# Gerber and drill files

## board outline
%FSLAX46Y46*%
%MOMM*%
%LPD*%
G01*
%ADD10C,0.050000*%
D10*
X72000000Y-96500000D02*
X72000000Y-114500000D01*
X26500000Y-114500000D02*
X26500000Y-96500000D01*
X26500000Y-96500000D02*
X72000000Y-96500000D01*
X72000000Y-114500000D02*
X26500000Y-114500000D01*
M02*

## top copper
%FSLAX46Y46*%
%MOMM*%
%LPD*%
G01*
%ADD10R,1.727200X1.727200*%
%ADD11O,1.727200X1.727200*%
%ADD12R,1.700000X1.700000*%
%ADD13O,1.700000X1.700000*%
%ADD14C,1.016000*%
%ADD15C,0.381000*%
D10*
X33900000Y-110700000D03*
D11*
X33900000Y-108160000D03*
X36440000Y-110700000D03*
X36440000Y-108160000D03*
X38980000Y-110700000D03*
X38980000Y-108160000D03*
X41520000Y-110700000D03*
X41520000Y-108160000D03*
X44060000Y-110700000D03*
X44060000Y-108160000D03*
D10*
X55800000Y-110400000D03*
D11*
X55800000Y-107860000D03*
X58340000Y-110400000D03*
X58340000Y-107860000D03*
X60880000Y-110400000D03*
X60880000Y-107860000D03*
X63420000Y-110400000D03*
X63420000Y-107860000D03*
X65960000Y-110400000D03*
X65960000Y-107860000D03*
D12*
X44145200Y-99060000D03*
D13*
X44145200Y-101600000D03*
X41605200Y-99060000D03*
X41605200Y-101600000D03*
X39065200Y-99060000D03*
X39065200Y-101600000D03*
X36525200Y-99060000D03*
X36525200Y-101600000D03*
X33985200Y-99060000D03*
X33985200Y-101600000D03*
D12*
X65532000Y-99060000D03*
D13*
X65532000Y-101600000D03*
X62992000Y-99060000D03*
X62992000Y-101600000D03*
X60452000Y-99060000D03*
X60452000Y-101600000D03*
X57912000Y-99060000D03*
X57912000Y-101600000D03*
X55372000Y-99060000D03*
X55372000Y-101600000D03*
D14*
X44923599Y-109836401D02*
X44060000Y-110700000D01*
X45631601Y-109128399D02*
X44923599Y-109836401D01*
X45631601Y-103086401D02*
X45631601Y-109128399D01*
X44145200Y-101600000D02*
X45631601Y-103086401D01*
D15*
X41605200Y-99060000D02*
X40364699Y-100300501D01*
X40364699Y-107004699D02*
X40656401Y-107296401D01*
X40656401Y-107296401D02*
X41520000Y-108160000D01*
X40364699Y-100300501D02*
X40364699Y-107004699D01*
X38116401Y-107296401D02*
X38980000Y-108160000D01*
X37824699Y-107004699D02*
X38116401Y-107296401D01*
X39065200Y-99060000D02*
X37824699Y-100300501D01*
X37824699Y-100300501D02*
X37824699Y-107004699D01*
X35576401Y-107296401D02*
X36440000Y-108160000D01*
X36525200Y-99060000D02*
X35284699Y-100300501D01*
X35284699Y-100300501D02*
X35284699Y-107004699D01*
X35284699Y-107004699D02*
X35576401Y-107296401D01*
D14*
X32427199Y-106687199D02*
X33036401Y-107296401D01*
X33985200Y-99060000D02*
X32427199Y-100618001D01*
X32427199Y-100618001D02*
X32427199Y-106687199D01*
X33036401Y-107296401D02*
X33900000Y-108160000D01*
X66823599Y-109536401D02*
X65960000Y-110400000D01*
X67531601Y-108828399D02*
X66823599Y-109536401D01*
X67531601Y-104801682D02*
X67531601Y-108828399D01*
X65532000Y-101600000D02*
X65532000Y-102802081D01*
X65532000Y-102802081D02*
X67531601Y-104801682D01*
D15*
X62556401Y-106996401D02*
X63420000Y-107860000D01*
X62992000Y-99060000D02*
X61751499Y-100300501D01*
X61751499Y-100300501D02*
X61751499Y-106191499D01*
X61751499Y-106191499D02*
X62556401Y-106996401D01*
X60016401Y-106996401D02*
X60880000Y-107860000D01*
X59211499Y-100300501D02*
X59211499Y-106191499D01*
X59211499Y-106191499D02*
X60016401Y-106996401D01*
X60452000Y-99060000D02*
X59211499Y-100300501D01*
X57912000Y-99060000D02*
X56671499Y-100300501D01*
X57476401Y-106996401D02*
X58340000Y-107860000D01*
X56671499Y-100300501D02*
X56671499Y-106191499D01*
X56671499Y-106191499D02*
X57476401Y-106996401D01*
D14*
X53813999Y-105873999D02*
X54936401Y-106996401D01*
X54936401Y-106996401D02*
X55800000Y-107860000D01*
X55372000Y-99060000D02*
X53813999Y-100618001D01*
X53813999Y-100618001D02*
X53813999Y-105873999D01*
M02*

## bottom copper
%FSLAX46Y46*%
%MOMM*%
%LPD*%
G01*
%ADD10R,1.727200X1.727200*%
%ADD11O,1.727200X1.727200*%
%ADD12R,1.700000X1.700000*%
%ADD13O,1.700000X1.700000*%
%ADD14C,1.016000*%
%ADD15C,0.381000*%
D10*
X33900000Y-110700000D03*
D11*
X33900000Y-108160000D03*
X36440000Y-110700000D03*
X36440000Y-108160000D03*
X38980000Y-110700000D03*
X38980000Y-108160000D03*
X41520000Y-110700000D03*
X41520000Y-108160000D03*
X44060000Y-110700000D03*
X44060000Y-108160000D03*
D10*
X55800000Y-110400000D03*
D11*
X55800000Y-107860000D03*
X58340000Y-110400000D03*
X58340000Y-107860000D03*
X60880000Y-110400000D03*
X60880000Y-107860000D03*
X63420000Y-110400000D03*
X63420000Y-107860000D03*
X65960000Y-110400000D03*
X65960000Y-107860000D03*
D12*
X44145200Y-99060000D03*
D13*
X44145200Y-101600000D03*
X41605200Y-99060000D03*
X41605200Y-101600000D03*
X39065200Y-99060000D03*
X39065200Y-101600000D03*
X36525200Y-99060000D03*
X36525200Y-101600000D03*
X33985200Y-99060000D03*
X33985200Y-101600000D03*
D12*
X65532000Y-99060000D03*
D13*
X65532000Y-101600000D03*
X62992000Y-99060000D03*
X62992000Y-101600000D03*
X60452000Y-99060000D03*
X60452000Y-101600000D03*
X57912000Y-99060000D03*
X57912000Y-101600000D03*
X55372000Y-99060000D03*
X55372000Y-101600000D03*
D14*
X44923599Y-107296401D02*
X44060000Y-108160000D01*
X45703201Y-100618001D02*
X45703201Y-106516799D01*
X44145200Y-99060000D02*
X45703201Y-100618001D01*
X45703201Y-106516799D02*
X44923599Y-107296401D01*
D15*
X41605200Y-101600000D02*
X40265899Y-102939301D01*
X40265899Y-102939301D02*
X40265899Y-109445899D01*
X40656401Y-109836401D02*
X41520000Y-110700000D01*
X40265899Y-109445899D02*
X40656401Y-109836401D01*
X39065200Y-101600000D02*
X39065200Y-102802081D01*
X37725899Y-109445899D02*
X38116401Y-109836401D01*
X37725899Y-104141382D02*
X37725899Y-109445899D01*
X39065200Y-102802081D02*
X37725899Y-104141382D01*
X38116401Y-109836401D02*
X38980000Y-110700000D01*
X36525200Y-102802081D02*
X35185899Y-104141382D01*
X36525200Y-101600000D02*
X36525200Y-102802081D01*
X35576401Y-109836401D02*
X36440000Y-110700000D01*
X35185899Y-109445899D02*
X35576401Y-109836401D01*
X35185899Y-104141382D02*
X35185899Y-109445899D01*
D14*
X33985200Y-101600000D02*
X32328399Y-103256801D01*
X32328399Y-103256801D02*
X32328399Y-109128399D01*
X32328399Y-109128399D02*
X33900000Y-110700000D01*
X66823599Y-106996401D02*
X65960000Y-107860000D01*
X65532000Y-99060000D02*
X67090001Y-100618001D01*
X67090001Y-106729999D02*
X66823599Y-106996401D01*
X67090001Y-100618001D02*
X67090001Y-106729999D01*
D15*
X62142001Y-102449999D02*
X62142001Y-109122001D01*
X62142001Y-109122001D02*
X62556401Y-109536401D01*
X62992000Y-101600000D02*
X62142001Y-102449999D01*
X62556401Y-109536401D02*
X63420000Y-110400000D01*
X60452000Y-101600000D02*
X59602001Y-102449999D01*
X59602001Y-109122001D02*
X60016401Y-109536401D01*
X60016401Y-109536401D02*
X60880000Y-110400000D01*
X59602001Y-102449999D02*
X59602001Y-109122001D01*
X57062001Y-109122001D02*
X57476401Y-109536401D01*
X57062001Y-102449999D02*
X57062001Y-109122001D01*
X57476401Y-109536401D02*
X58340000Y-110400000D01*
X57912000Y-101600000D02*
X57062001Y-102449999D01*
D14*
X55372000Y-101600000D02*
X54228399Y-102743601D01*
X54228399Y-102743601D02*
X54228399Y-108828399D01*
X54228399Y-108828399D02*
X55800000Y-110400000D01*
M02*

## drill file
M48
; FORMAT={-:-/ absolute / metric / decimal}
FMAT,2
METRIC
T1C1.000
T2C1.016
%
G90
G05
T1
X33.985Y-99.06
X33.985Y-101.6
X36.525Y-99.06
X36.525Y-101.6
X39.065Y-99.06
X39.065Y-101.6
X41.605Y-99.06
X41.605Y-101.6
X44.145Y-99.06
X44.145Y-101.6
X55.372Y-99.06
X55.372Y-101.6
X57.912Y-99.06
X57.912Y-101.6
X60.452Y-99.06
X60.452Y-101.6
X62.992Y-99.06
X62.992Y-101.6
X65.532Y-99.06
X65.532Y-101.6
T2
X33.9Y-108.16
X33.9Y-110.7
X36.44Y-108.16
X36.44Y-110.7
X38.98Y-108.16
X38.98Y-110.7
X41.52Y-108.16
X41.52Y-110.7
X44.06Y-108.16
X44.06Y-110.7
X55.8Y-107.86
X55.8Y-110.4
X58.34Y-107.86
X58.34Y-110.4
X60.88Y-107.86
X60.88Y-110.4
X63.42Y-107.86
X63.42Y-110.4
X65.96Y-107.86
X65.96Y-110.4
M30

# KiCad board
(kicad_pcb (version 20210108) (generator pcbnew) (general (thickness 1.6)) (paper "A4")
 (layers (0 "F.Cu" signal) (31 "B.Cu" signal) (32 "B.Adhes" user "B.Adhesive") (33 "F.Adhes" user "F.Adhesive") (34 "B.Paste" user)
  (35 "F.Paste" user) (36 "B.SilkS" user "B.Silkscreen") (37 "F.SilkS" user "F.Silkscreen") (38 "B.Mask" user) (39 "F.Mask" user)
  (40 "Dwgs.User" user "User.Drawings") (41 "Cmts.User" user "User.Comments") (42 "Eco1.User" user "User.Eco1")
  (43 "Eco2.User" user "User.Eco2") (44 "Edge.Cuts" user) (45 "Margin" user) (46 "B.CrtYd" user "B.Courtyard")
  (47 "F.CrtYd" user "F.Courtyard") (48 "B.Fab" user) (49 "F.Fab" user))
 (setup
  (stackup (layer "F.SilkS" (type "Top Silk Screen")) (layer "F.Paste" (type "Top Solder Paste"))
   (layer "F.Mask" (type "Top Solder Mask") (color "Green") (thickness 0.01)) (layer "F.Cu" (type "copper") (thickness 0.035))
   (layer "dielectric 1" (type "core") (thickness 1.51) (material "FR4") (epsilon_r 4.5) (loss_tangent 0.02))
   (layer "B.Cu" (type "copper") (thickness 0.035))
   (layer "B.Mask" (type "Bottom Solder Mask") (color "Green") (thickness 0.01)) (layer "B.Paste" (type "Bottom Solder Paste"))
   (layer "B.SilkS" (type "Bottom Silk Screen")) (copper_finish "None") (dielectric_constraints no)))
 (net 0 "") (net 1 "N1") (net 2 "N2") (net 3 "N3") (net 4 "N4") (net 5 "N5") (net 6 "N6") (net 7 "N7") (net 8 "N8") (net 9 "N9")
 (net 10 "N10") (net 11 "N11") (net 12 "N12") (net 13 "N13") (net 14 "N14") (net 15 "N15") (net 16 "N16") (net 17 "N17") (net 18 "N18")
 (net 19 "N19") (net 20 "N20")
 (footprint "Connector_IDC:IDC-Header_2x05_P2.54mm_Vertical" (layer "F.Cu") (at 33.9 110.7 90)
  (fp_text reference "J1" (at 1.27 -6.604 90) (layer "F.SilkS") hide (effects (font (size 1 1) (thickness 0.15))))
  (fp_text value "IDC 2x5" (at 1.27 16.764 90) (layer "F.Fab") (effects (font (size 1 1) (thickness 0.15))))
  (pad "1" thru_hole rect (at 0 0 90) (locked) (size 1.7272 1.7272) (drill 1.016) (layers *.Cu *.Mask) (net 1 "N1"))
  (pad "2" thru_hole oval (at 2.54 0 90) (locked) (size 1.7272 1.7272) (drill 1.016) (layers *.Cu *.Mask) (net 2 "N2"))
  (pad "3" thru_hole oval (at 0 2.54 90) (locked) (size 1.7272 1.7272) (drill 1.016) (layers *.Cu *.Mask) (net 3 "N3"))
  (pad "4" thru_hole oval (at 2.54 2.54 90) (locked) (size 1.7272 1.7272) (drill 1.016) (layers *.Cu *.Mask) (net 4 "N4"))
  (pad "5" thru_hole oval (at 0 5.08 90) (locked) (size 1.7272 1.7272) (drill 1.016) (layers *.Cu *.Mask) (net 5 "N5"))
  (pad "6" thru_hole oval (at 2.54 5.08 90) (locked) (size 1.7272 1.7272) (drill 1.016) (layers *.Cu *.Mask) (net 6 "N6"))
  (pad "7" thru_hole oval (at 0 7.62 90) (locked) (size 1.7272 1.7272) (drill 1.016) (layers *.Cu *.Mask) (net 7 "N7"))
  (pad "8" thru_hole oval (at 2.54 7.62 90) (locked) (size 1.7272 1.7272) (drill 1.016) (layers *.Cu *.Mask) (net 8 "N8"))
  (pad "9" thru_hole oval (at 0 10.16 90) (locked) (size 1.7272 1.7272) (drill 1.016) (layers *.Cu *.Mask) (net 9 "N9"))
  (pad "10" thru_hole oval (at 2.54 10.16 90) (locked) (size 1.7272 1.7272) (drill 1.016) (layers *.Cu *.Mask) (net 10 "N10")))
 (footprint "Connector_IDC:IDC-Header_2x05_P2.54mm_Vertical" (layer "F.Cu") (at 55.8 110.4 90)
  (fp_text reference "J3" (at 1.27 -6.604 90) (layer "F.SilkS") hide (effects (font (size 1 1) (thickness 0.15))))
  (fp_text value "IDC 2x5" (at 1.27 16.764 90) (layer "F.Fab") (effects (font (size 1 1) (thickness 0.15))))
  (pad "1" thru_hole rect (at 0 0 90) (locked) (size 1.7272 1.7272) (drill 1.016) (layers *.Cu *.Mask) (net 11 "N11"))
  (pad "2" thru_hole oval (at 2.54 0 90) (locked) (size 1.7272 1.7272) (drill 1.016) (layers *.Cu *.Mask) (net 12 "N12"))
  (pad "3" thru_hole oval (at 0 2.54 90) (locked) (size 1.7272 1.7272) (drill 1.016) (layers *.Cu *.Mask) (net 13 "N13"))
  (pad "4" thru_hole oval (at 2.54 2.54 90) (locked) (size 1.7272 1.7272) (drill 1.016) (layers *.Cu *.Mask) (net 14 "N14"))
  (pad "5" thru_hole oval (at 0 5.08 90) (locked) (size 1.7272 1.7272) (drill 1.016) (layers *.Cu *.Mask) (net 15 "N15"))
  (pad "6" thru_hole oval (at 2.54 5.08 90) (locked) (size 1.7272 1.7272) (drill 1.016) (layers *.Cu *.Mask) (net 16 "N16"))
  (pad "7" thru_hole oval (at 0 7.62 90) (locked) (size 1.7272 1.7272) (drill 1.016) (layers *.Cu *.Mask) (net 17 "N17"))
  (pad "8" thru_hole oval (at 2.54 7.62 90) (locked) (size 1.7272 1.7272) (drill 1.016) (layers *.Cu *.Mask) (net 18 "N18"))
  (pad "9" thru_hole oval (at 0 10.16 90) (locked) (size 1.7272 1.7272) (drill 1.016) (layers *.Cu *.Mask) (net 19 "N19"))
  (pad "10" thru_hole oval (at 2.54 10.16 90) (locked) (size 1.7272 1.7272) (drill 1.016) (layers *.Cu *.Mask) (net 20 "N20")))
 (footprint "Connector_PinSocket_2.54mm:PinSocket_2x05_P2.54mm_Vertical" (layer "B.Cu") (at 44.1452 99.06 90)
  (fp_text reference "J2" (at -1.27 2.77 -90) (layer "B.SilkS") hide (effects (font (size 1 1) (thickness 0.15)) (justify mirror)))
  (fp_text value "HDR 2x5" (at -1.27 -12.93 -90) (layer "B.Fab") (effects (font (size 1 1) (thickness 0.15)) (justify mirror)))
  (pad "1" thru_hole rect (at 0 0 90) (locked) (size 1.7 1.7) (drill 1) (layers *.Cu *.Mask) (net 10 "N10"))
  (pad "2" thru_hole oval (at -2.54 0 90) (locked) (size 1.7 1.7) (drill 1) (layers *.Cu *.Mask) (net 9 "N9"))
  (pad "3" thru_hole oval (at 0 -2.54 90) (locked) (size 1.7 1.7) (drill 1) (layers *.Cu *.Mask) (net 8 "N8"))
  (pad "4" thru_hole oval (at -2.54 -2.54 90) (locked) (size 1.7 1.7) (drill 1) (layers *.Cu *.Mask) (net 7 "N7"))
  (pad "5" thru_hole oval (at 0 -5.08 90) (locked) (size 1.7 1.7) (drill 1) (layers *.Cu *.Mask) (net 6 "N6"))
  (pad "6" thru_hole oval (at -2.54 -5.08 90) (locked) (size 1.7 1.7) (drill 1) (layers *.Cu *.Mask) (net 5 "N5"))
  (pad "7" thru_hole oval (at 0 -7.62 90) (locked) (size 1.7 1.7) (drill 1) (layers *.Cu *.Mask) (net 4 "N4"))
  (pad "8" thru_hole oval (at -2.54 -7.62 90) (locked) (size 1.7 1.7) (drill 1) (layers *.Cu *.Mask) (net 3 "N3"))
  (pad "9" thru_hole oval (at 0 -10.16 90) (locked) (size 1.7 1.7) (drill 1) (layers *.Cu *.Mask) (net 2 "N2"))
  (pad "10" thru_hole oval (at -2.54 -10.16 90) (locked) (size 1.7 1.7) (drill 1) (layers *.Cu *.Mask) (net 1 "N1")))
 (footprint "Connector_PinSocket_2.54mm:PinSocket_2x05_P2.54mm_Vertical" (layer "B.Cu") (at 65.532 99.06 90)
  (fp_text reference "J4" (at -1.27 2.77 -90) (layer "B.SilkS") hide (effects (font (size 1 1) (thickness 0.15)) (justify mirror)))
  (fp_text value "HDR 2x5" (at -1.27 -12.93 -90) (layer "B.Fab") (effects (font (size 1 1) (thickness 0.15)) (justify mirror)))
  (pad "1" thru_hole rect (at 0 0 90) (locked) (size 1.7 1.7) (drill 1) (layers *.Cu *.Mask) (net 20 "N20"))
  (pad "2" thru_hole oval (at -2.54 0 90) (locked) (size 1.7 1.7) (drill 1) (layers *.Cu *.Mask) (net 19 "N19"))
  (pad "3" thru_hole oval (at 0 -2.54 90) (locked) (size 1.7 1.7) (drill 1) (layers *.Cu *.Mask) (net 18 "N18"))
  (pad "4" thru_hole oval (at -2.54 -2.54 90) (locked) (size 1.7 1.7) (drill 1) (layers *.Cu *.Mask) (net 17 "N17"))
  (pad "5" thru_hole oval (at 0 -5.08 90) (locked) (size 1.7 1.7) (drill 1) (layers *.Cu *.Mask) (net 16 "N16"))
  (pad "6" thru_hole oval (at -2.54 -5.08 90) (locked) (size 1.7 1.7) (drill 1) (layers *.Cu *.Mask) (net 15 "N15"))
  (pad "7" thru_hole oval (at 0 -7.62 90) (locked) (size 1.7 1.7) (drill 1) (layers *.Cu *.Mask) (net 14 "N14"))
  (pad "8" thru_hole oval (at -2.54 -7.62 90) (locked) (size 1.7 1.7) (drill 1) (layers *.Cu *.Mask) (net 13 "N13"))
  (pad "9" thru_hole oval (at 0 -10.16 90) (locked) (size 1.7 1.7) (drill 1) (layers *.Cu *.Mask) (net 12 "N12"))
  (pad "10" thru_hole oval (at -2.54 -10.16 90) (locked) (size 1.7 1.7) (drill 1) (layers *.Cu *.Mask) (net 11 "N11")))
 (gr_line (start 72 96.5) (end 72 114.5) (layer "Edge.Cuts") (width 0.05))
 (gr_line (start 26.5 114.5) (end 26.5 96.5) (layer "Edge.Cuts") (width 0.05))
 (gr_line (start 26.5 96.5) (end 72 96.5) (layer "Edge.Cuts") (width 0.05))
 (gr_line (start 72 114.5) (end 26.5 114.5) (layer "Edge.Cuts") (width 0.05))
 (segment (start 44.923599 107.296401) (end 44.06 108.16) (width 1.016) (layer "B.Cu") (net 10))
 (segment (start 45.703201 100.618001) (end 45.703201 106.516799) (width 1.016) (layer "B.Cu") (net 10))
 (segment (start 44.1452 99.06) (end 45.703201 100.618001) (width 1.016) (layer "B.Cu") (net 10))
 (segment (start 45.703201 106.516799) (end 44.923599 107.296401) (width 1.016) (layer "B.Cu") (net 10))
 (segment (start 44.923599 109.836401) (end 44.06 110.7) (width 1.016) (layer "F.Cu") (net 9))
 (segment (start 45.631601 109.128399) (end 44.923599 109.836401) (width 1.016) (layer "F.Cu") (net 9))
 (segment (start 45.631601 103.086401) (end 45.631601 109.128399) (width 1.016) (layer "F.Cu") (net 9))
 (segment (start 44.1452 101.6) (end 45.631601 103.086401) (width 1.016) (layer "F.Cu") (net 9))
 (segment (start 41.6052 99.06) (end 40.364699 100.300501) (width 0.381) (layer "F.Cu") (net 8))
 (segment (start 40.364699 107.004699) (end 40.656401 107.296401) (width 0.381) (layer "F.Cu") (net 8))
 (segment (start 40.656401 107.296401) (end 41.52 108.16) (width 0.381) (layer "F.Cu") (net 8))
 (segment (start 40.364699 100.300501) (end 40.364699 107.004699) (width 0.381) (layer "F.Cu") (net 8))
 (segment (start 41.6052 101.6) (end 40.265899 102.939301) (width 0.381) (layer "B.Cu") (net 7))
 (segment (start 40.265899 102.939301) (end 40.265899 109.445899) (width 0.381) (layer "B.Cu") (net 7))
 (segment (start 40.656401 109.836401) (end 41.52 110.7) (width 0.381) (layer "B.Cu") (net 7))
 (segment (start 40.265899 109.445899) (end 40.656401 109.836401) (width 0.381) (layer "B.Cu") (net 7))
 (segment (start 38.116401 107.296401) (end 38.98 108.16) (width 0.381) (layer "F.Cu") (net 6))
 (segment (start 37.824699 107.004699) (end 38.116401 107.296401) (width 0.381) (layer "F.Cu") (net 6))
 (segment (start 39.0652 99.06) (end 37.824699 100.300501) (width 0.381) (layer "F.Cu") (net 6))
 (segment (start 37.824699 100.300501) (end 37.824699 107.004699) (width 0.381) (layer "F.Cu") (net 6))
 (segment (start 39.0652 101.6) (end 39.0652 102.802081) (width 0.381) (layer "B.Cu") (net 5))
 (segment (start 37.725899 109.445899) (end 38.116401 109.836401) (width 0.381) (layer "B.Cu") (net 5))
 (segment (start 37.725899 104.141382) (end 37.725899 109.445899) (width 0.381) (layer "B.Cu") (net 5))
 (segment (start 39.0652 102.802081) (end 37.725899 104.141382) (width 0.381) (layer "B.Cu") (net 5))
 (segment (start 38.116401 109.836401) (end 38.98 110.7) (width 0.381) (layer "B.Cu") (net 5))
 (segment (start 35.576401 107.296401) (end 36.44 108.16) (width 0.381) (layer "F.Cu") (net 4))
 (segment (start 36.5252 99.06) (end 35.284699 100.300501) (width 0.381) (layer "F.Cu") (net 4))
 (segment (start 35.284699 100.300501) (end 35.284699 107.004699) (width 0.381) (layer "F.Cu") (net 4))
 (segment (start 35.284699 107.004699) (end 35.576401 107.296401) (width 0.381) (layer "F.Cu") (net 4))
 (segment (start 36.5252 102.802081) (end 35.185899 104.141382) (width 0.381) (layer "B.Cu") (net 3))
 (segment (start 36.5252 101.6) (end 36.5252 102.802081) (width 0.381) (layer "B.Cu") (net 3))
 (segment (start 35.576401 109.836401) (end 36.44 110.7) (width 0.381) (layer "B.Cu") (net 3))
 (segment (start 35.185899 109.445899) (end 35.576401 109.836401) (width 0.381) (layer "B.Cu") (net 3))
 (segment (start 35.185899 104.141382) (end 35.185899 109.445899) (width 0.381) (layer "B.Cu") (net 3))
 (segment (start 32.427199 106.687199) (end 33.036401 107.296401) (width 1.016) (layer "F.Cu") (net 2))
 (segment (start 33.9852 99.06) (end 32.427199 100.618001) (width 1.016) (layer "F.Cu") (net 2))
 (segment (start 32.427199 100.618001) (end 32.427199 106.687199) (width 1.016) (layer "F.Cu") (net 2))
 (segment (start 33.036401 107.296401) (end 33.9 108.16) (width 1.016) (layer "F.Cu") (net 2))
 (segment (start 33.9852 101.6) (end 32.328399 103.256801) (width 1.016) (layer "B.Cu") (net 1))
 (segment (start 32.328399 103.256801) (end 32.328399 109.128399) (width 1.016) (layer "B.Cu") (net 1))
 (segment (start 32.328399 109.128399) (end 33.9 110.7) (width 1.016) (layer "B.Cu") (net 1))
 (segment (start 66.823599 106.996401) (end 65.96 107.86) (width 1.016) (layer "B.Cu") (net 20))
 (segment (start 65.532 99.06) (end 67.090001 100.618001) (width 1.016) (layer "B.Cu") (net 20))
 (segment (start 67.090001 106.729999) (end 66.823599 106.996401) (width 1.016) (layer "B.Cu") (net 20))
 (segment (start 67.090001 100.618001) (end 67.090001 106.729999) (width 1.016) (layer "B.Cu") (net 20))
 (segment (start 66.823599 109.536401) (end 65.96 110.4) (width 1.016) (layer "F.Cu") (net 19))
 (segment (start 67.531601 108.828399) (end 66.823599 109.536401) (width 1.016) (layer "F.Cu") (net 19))
 (segment (start 67.531601 104.801682) (end 67.531601 108.828399) (width 1.016) (layer "F.Cu") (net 19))
 (segment (start 65.532 101.6) (end 65.532 102.802081) (width 1.016) (layer "F.Cu") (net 19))
 (segment (start 65.532 102.802081) (end 67.531601 104.801682) (width 1.016) (layer "F.Cu") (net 19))
 (segment (start 62.556401 106.996401) (end 63.42 107.86) (width 0.381) (layer "F.Cu") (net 18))
 (segment (start 62.992 99.06) (end 61.751499 100.300501) (width 0.381) (layer "F.Cu") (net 18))
 (segment (start 61.751499 100.300501) (end 61.751499 106.191499) (width 0.381) (layer "F.Cu") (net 18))
 (segment (start 61.751499 106.191499) (end 62.556401 106.996401) (width 0.381) (layer "F.Cu") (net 18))
 (segment (start 62.142001 102.449999) (end 62.142001 109.122001) (width 0.381) (layer "B.Cu") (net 17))
 (segment (start 62.142001 109.122001) (end 62.556401 109.536401) (width 0.381) (layer "B.Cu") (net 17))
 (segment (start 62.992 101.6) (end 62.142001 102.449999) (width 0.381) (layer "B.Cu") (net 17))
 (segment (start 62.556401 109.536401) (end 63.42 110.4) (width 0.381) (layer "B.Cu") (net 17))
 (segment (start 60.016401 106.996401) (end 60.88 107.86) (width 0.381) (layer "F.Cu") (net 16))
 (segment (start 59.211499 100.300501) (end 59.211499 106.191499) (width 0.381) (layer "F.Cu") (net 16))
 (segment (start 59.211499 106.191499) (end 60.016401 106.996401) (width 0.381) (layer "F.Cu") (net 16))
 (segment (start 60.452 99.06) (end 59.211499 100.300501) (width 0.381) (layer "F.Cu") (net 16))
 (segment (start 60.452 101.6) (end 59.602001 102.449999) (width 0.381) (layer "B.Cu") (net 15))
 (segment (start 59.602001 109.122001) (end 60.016401 109.536401) (width 0.381) (layer "B.Cu") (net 15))
 (segment (start 60.016401 109.536401) (end 60.88 110.4) (width 0.381) (layer "B.Cu") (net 15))
 (segment (start 59.602001 102.449999) (end 59.602001 109.122001) (width 0.381) (layer "B.Cu") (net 15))
 (segment (start 57.912 99.06) (end 56.671499 100.300501) (width 0.381) (layer "F.Cu") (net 14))
 (segment (start 57.476401 106.996401) (end 58.34 107.86) (width 0.381) (layer "F.Cu") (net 14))
 (segment (start 56.671499 100.300501) (end 56.671499 106.191499) (width 0.381) (layer "F.Cu") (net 14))
 (segment (start 56.671499 106.191499) (end 57.476401 106.996401) (width 0.381) (layer "F.Cu") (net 14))
 (segment (start 57.062001 109.122001) (end 57.476401 109.536401) (width 0.381) (layer "B.Cu") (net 13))
 (segment (start 57.062001 102.449999) (end 57.062001 109.122001) (width 0.381) (layer "B.Cu") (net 13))
 (segment (start 57.476401 109.536401) (end 58.34 110.4) (width 0.381) (layer "B.Cu") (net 13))
 (segment (start 57.912 101.6) (end 57.062001 102.449999) (width 0.381) (layer "B.Cu") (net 13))
 (segment (start 53.813999 105.873999) (end 54.936401 106.996401) (width 1.016) (layer "F.Cu") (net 12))
 (segment (start 54.936401 106.996401) (end 55.8 107.86) (width 1.016) (layer "F.Cu") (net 12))
 (segment (start 55.372 99.06) (end 53.813999 100.618001) (width 1.016) (layer "F.Cu") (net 12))
 (segment (start 53.813999 100.618001) (end 53.813999 105.873999) (width 1.016) (layer "F.Cu") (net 12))
 (segment (start 55.372 101.6) (end 54.228399 102.743601) (width 1.016) (layer "B.Cu") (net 11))
 (segment (start 54.228399 102.743601) (end 54.228399 108.828399) (width 1.016) (layer "B.Cu") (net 11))
 (segment (start 54.228399 108.828399) (end 55.8 110.4) (width 1.016) (layer "B.Cu") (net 11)))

